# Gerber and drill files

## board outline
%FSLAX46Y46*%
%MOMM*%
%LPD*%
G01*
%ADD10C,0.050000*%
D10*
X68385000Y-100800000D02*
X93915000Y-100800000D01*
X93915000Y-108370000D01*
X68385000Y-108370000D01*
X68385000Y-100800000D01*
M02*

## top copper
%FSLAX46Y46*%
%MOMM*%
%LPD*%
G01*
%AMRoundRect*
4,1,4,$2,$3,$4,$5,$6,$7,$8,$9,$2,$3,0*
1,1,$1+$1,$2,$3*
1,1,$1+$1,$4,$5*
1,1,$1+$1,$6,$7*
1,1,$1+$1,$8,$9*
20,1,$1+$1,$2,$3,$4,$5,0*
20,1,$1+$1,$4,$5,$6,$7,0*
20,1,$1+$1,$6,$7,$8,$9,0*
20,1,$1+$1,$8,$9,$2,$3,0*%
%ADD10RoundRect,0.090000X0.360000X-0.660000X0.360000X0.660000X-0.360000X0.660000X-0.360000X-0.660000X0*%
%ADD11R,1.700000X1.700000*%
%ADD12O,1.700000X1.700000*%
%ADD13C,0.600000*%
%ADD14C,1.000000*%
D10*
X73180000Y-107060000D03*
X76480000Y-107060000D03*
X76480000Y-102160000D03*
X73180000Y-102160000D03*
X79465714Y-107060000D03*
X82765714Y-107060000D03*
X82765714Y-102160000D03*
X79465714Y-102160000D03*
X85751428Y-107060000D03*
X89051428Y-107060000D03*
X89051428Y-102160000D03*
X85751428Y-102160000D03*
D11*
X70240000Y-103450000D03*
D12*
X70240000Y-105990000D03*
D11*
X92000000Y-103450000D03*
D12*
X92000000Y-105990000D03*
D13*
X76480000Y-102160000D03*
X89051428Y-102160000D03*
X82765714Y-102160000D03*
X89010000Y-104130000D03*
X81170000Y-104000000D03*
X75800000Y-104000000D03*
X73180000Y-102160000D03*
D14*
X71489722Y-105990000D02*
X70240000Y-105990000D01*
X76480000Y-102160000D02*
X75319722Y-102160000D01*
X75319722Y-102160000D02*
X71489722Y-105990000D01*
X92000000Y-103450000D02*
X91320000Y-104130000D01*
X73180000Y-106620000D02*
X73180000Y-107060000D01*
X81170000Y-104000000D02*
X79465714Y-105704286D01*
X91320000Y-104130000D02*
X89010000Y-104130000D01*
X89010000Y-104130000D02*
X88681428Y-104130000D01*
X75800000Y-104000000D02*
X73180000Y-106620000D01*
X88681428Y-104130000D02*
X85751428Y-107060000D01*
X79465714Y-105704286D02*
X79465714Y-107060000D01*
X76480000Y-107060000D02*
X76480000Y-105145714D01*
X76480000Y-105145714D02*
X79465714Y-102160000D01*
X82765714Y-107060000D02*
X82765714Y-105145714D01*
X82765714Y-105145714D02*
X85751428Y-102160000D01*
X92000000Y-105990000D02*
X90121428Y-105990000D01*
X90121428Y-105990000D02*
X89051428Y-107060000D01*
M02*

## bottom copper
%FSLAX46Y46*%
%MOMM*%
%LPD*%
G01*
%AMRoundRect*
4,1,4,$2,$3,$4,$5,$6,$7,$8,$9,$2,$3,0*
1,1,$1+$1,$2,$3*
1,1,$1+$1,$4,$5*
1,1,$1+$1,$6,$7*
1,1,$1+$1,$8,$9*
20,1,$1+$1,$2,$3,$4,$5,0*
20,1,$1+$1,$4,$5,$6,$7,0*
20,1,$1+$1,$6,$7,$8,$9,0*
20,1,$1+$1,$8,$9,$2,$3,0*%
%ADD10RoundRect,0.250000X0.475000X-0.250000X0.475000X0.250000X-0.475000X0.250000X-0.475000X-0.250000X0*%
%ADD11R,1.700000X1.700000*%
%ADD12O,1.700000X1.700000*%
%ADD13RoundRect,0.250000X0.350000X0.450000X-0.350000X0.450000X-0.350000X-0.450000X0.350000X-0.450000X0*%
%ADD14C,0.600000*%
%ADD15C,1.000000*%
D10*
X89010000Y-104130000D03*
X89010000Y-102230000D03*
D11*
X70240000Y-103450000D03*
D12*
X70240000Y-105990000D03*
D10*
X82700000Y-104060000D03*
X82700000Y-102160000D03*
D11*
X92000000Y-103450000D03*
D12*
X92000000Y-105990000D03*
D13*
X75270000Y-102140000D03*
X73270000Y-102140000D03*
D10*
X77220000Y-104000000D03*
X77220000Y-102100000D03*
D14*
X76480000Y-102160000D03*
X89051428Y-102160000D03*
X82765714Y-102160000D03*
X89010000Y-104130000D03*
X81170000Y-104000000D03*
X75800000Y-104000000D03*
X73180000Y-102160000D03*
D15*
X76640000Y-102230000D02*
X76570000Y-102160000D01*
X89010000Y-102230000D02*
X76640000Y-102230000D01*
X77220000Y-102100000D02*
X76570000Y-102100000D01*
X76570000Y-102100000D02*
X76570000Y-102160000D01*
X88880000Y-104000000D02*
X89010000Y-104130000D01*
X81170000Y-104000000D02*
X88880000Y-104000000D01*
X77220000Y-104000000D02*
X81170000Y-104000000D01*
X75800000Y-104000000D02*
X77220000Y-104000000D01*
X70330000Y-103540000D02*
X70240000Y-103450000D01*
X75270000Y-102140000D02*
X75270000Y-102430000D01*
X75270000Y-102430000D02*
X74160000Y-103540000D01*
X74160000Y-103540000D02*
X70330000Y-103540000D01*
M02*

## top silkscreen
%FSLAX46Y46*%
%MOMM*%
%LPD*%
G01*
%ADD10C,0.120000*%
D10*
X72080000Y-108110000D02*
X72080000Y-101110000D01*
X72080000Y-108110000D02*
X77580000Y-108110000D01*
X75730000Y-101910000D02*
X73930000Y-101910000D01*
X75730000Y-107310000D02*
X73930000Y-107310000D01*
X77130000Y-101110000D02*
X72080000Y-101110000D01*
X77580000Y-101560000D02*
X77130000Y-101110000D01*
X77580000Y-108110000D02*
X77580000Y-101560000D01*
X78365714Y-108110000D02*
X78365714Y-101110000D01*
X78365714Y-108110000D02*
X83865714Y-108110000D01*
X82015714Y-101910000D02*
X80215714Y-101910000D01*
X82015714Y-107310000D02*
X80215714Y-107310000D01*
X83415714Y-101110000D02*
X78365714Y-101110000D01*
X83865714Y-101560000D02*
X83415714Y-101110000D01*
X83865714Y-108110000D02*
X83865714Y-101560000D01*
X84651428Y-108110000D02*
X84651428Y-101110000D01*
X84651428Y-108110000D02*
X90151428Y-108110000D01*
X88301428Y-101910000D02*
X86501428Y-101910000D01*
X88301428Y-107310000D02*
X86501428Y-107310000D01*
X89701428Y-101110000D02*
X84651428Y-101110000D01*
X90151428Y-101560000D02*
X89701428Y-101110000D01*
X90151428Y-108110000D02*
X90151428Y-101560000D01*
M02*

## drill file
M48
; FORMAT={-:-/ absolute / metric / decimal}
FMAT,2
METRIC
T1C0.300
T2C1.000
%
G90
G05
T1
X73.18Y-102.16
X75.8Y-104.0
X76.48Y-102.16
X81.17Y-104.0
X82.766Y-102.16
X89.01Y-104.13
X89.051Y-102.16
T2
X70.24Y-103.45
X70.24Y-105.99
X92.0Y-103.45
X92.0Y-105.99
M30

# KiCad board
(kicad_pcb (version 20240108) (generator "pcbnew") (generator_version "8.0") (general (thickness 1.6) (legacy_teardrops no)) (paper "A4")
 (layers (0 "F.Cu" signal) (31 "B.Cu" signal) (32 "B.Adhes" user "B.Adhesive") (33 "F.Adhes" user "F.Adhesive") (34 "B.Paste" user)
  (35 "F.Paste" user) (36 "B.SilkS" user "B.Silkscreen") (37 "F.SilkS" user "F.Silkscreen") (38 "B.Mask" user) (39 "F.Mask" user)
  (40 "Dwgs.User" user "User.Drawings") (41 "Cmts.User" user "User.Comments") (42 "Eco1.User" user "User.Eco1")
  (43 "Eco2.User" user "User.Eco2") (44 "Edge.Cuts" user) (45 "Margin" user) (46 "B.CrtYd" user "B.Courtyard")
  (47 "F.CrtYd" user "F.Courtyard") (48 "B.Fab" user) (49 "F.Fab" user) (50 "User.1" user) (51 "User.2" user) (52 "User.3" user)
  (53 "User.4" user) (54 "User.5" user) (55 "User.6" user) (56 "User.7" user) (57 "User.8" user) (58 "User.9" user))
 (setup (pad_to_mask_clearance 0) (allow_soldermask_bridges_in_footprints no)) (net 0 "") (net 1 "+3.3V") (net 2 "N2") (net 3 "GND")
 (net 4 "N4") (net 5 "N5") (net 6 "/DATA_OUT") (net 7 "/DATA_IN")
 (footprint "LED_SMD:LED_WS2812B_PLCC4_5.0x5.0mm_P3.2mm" (layer "F.Cu") (at 74.83 104.61 90)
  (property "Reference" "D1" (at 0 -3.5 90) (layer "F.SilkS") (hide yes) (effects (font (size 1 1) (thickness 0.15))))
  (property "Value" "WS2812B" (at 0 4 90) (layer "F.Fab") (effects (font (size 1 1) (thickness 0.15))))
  (fp_line (start -3.5 -2.75) (end 3.5 -2.75) (stroke (width 0.12) (type solid)) (layer "F.SilkS"))
  (fp_line (start -3.5 -2.75) (end -3.5 2.75) (stroke (width 0.12) (type default)) (layer "F.SilkS"))
  (fp_line (start 2.7 0.9) (end 2.7 -0.9) (stroke (width 0.12) (type default)) (layer "F.SilkS"))
  (fp_line (start -2.7 0.9) (end -2.7 -0.9) (stroke (width 0.12) (type default)) (layer "F.SilkS"))
  (fp_line (start 3.5 2.3) (end 3.5 -2.75) (stroke (width 0.12) (type default)) (layer "F.SilkS"))
  (fp_line (start 3.05 2.75) (end 3.5 2.3) (stroke (width 0.12) (type default)) (layer "F.SilkS"))
  (fp_line (start -3.5 2.75) (end 3.05 2.75) (stroke (width 0.12) (type solid)) (layer "F.SilkS"))
  (pad "1" smd roundrect (at -2.45 -1.65 90) (size 1.5 0.9) (layers "F.Cu" "F.Paste" "F.Mask") (roundrect_rratio 0.1) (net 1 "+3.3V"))
  (pad "2" smd roundrect (at -2.45 1.65 90) (size 1.5 0.9) (layers "F.Cu" "F.Paste" "F.Mask") (roundrect_rratio 0.1) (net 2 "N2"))
  (pad "3" smd roundrect (at 2.45 1.65 90) (size 1.5 0.9) (layers "F.Cu" "F.Paste" "F.Mask") (roundrect_rratio 0.1) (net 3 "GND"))
  (pad "4" smd roundrect (at 2.45 -1.65 90) (size 1.5 0.9) (layers "F.Cu" "F.Paste" "F.Mask") (roundrect_rratio 0.1) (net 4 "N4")))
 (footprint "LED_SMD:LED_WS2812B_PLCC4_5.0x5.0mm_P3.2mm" (layer "F.Cu") (at 81.115714 104.61 90)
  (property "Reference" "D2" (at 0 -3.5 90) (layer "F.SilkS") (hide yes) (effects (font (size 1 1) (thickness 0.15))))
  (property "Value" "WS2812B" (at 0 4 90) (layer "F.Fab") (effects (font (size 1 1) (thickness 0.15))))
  (fp_line (start -3.5 -2.75) (end 3.5 -2.75) (stroke (width 0.12) (type solid)) (layer "F.SilkS"))
  (fp_line (start -3.5 -2.75) (end -3.5 2.75) (stroke (width 0.12) (type default)) (layer "F.SilkS"))
  (fp_line (start 2.7 0.9) (end 2.7 -0.9) (stroke (width 0.12) (type default)) (layer "F.SilkS"))
  (fp_line (start -2.7 0.9) (end -2.7 -0.9) (stroke (width 0.12) (type default)) (layer "F.SilkS"))
  (fp_line (start 3.5 2.3) (end 3.5 -2.75) (stroke (width 0.12) (type default)) (layer "F.SilkS"))
  (fp_line (start 3.05 2.75) (end 3.5 2.3) (stroke (width 0.12) (type default)) (layer "F.SilkS"))
  (fp_line (start -3.5 2.75) (end 3.05 2.75) (stroke (width 0.12) (type solid)) (layer "F.SilkS"))
  (pad "1" smd roundrect (at -2.45 -1.65 90) (size 1.5 0.9) (layers "F.Cu" "F.Paste" "F.Mask") (roundrect_rratio 0.1) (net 1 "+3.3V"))
  (pad "2" smd roundrect (at -2.45 1.65 90) (size 1.5 0.9) (layers "F.Cu" "F.Paste" "F.Mask") (roundrect_rratio 0.1) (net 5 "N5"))
  (pad "3" smd roundrect (at 2.45 1.65 90) (size 1.5 0.9) (layers "F.Cu" "F.Paste" "F.Mask") (roundrect_rratio 0.1) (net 3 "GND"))
  (pad "4" smd roundrect (at 2.45 -1.65 90) (size 1.5 0.9) (layers "F.Cu" "F.Paste" "F.Mask") (roundrect_rratio 0.1) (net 2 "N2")))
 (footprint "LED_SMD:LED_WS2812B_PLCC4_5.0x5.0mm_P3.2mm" (layer "F.Cu") (at 87.401428 104.61 90)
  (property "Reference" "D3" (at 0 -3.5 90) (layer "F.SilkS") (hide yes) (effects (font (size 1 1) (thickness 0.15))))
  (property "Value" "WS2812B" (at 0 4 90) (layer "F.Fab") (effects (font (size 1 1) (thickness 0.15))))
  (fp_line (start -3.5 -2.75) (end 3.5 -2.75) (stroke (width 0.12) (type solid)) (layer "F.SilkS"))
  (fp_line (start -3.5 -2.75) (end -3.5 2.75) (stroke (width 0.12) (type default)) (layer "F.SilkS"))
  (fp_line (start 2.7 0.9) (end 2.7 -0.9) (stroke (width 0.12) (type default)) (layer "F.SilkS"))
  (fp_line (start -2.7 0.9) (end -2.7 -0.9) (stroke (width 0.12) (type default)) (layer "F.SilkS"))
  (fp_line (start 3.5 2.3) (end 3.5 -2.75) (stroke (width 0.12) (type default)) (layer "F.SilkS"))
  (fp_line (start 3.05 2.75) (end 3.5 2.3) (stroke (width 0.12) (type default)) (layer "F.SilkS"))
  (fp_line (start -3.5 2.75) (end 3.05 2.75) (stroke (width 0.12) (type solid)) (layer "F.SilkS"))
  (pad "1" smd roundrect (at -2.45 -1.65 90) (size 1.5 0.9) (layers "F.Cu" "F.Paste" "F.Mask") (roundrect_rratio 0.1) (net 1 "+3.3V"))
  (pad "2" smd roundrect (at -2.45 1.65 90) (size 1.5 0.9) (layers "F.Cu" "F.Paste" "F.Mask") (roundrect_rratio 0.1) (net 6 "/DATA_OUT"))
  (pad "3" smd roundrect (at 2.45 1.65 90) (size 1.5 0.9) (layers "F.Cu" "F.Paste" "F.Mask") (roundrect_rratio 0.1) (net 3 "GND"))
  (pad "4" smd roundrect (at 2.45 -1.65 90) (size 1.5 0.9) (layers "F.Cu" "F.Paste" "F.Mask") (roundrect_rratio 0.1) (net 5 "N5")))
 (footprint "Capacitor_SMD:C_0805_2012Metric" (layer "B.Cu") (at 89.01 103.18 90)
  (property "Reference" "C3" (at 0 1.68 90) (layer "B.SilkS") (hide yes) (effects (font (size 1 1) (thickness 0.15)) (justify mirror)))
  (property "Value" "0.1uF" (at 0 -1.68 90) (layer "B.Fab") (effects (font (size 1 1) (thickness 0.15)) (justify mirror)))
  (pad "1" smd roundrect (at -0.95 0 90) (size 1 1.45) (layers "B.Cu" "B.Paste" "B.Mask") (roundrect_rratio 0.25) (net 1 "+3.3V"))
  (pad "2" smd roundrect (at 0.95 0 90) (size 1 1.45) (layers "B.Cu" "B.Paste" "B.Mask") (roundrect_rratio 0.25) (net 3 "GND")))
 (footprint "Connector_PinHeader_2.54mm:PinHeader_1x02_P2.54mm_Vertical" (layer "B.Cu") (at 70.24 103.45 180)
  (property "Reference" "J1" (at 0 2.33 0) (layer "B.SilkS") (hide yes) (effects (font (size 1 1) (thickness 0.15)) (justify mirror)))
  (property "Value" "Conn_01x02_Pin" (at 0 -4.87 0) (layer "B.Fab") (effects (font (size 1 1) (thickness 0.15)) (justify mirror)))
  (pad "1" thru_hole rect (at 0 0 180) (size 1.7 1.7) (drill 1) (layers "*.Cu" "*.Mask") (remove_unused_layers no) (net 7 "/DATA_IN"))
  (pad "2" thru_hole oval (at 0 -2.54 180) (size 1.7 1.7) (drill 1) (layers "*.Cu" "*.Mask") (remove_unused_layers no) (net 3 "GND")))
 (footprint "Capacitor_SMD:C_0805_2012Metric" (layer "B.Cu") (at 82.7 103.11 90)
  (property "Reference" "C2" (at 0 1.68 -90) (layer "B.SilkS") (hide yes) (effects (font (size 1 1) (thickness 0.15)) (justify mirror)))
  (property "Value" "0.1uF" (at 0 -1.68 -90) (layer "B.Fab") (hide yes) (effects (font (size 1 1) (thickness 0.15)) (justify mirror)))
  (pad "1" smd roundrect (at -0.95 0 90) (size 1 1.45) (layers "B.Cu" "B.Paste" "B.Mask") (roundrect_rratio 0.25) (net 1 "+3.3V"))
  (pad "2" smd roundrect (at 0.95 0 90) (size 1 1.45) (layers "B.Cu" "B.Paste" "B.Mask") (roundrect_rratio 0.25) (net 3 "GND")))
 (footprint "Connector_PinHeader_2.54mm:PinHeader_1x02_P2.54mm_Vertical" (layer "B.Cu") (at 92 103.45 180)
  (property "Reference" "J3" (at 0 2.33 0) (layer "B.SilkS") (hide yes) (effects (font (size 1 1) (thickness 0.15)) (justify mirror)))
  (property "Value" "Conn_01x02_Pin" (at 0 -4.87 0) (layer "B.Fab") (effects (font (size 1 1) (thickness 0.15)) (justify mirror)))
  (pad "1" thru_hole rect (at 0 0 180) (size 1.7 1.7) (drill 1) (layers "*.Cu" "*.Mask") (remove_unused_layers no) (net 1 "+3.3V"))
  (pad "2" thru_hole oval (at 0 -2.54 180) (size 1.7 1.7) (drill 1) (layers "*.Cu" "*.Mask") (remove_unused_layers no) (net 6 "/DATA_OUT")))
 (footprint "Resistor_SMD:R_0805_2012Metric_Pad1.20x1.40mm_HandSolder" (layer "B.Cu") (at 74.27 102.14 180)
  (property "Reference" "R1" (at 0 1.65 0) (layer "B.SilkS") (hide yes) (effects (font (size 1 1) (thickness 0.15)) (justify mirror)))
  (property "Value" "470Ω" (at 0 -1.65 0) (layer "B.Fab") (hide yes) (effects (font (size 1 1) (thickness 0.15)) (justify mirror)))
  (pad "1" smd roundrect (at -1 0 180) (size 1.2 1.4) (layers "B.Cu" "B.Paste" "B.Mask") (roundrect_rratio 0.208333) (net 7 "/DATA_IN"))
  (pad "2" smd roundrect (at 1 0 180) (size 1.2 1.4) (layers "B.Cu" "B.Paste" "B.Mask") (roundrect_rratio 0.208333) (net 4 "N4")))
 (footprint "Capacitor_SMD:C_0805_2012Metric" (layer "B.Cu") (at 77.22 103.05 90)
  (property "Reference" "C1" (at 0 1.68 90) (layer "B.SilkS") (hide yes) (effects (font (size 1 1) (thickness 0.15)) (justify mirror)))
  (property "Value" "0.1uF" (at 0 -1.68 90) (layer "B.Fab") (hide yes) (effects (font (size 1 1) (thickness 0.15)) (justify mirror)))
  (pad "1" smd roundrect (at -0.95 0 90) (size 1 1.45) (layers "B.Cu" "B.Paste" "B.Mask") (roundrect_rratio 0.25) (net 1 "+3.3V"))
  (pad "2" smd roundrect (at 0.95 0 90) (size 1 1.45) (layers "B.Cu" "B.Paste" "B.Mask") (roundrect_rratio 0.25) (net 3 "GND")))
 (gr_rect (start 68.385 100.8) (end 93.915 108.37) (stroke (width 0.05) (type default)) (fill none) (layer "Edge.Cuts"))
 (segment (start 71.489722 105.99) (end 70.24 105.99) (width 1) (layer "F.Cu") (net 3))
 (segment (start 76.48 102.16) (end 75.319722 102.16) (width 1) (layer "F.Cu") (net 3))
 (segment (start 75.319722 102.16) (end 71.489722 105.99) (width 1) (layer "F.Cu") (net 3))
 (via (at 76.48 102.16) (size 0.6) (drill 0.3) (layers "F.Cu" "B.Cu") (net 3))
 (via (at 89.051428 102.16) (size 0.6) (drill 0.3) (layers "F.Cu" "B.Cu") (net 3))
 (via (at 82.765714 102.16) (size 0.6) (drill 0.3) (layers "F.Cu" "B.Cu") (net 3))
 (segment (start 76.64 102.23) (end 76.57 102.16) (width 1) (layer "B.Cu") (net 3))
 (segment (start 89.01 102.23) (end 76.64 102.23) (width 1) (layer "B.Cu") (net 3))
 (segment (start 77.22 102.1) (end 76.57 102.1) (width 1) (layer "B.Cu") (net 3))
 (segment (start 76.57 102.1) (end 76.57 102.16) (width 1) (layer "B.Cu") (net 3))
 (segment (start 92 103.45) (end 91.32 104.13) (width 1) (layer "F.Cu") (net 1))
 (segment (start 73.18 106.62) (end 73.18 107.06) (width 1) (layer "F.Cu") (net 1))
 (segment (start 81.17 104) (end 79.465714 105.704286) (width 1) (layer "F.Cu") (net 1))
 (segment (start 91.32 104.13) (end 89.01 104.13) (width 1) (layer "F.Cu") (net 1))
 (segment (start 89.01 104.13) (end 88.681428 104.13) (width 1) (layer "F.Cu") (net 1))
 (segment (start 75.8 104) (end 73.18 106.62) (width 1) (layer "F.Cu") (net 1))
 (segment (start 88.681428 104.13) (end 85.751428 107.06) (width 1) (layer "F.Cu") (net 1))
 (segment (start 79.465714 105.704286) (end 79.465714 107.06) (width 1) (layer "F.Cu") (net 1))
 (via (at 89.01 104.13) (size 0.6) (drill 0.3) (layers "F.Cu" "B.Cu") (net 1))
 (via (at 81.17 104) (size 0.6) (drill 0.3) (layers "F.Cu" "B.Cu") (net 1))
 (via (at 75.8 104) (size 0.6) (drill 0.3) (layers "F.Cu" "B.Cu") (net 1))
 (segment (start 88.88 104) (end 89.01 104.13) (width 1) (layer "B.Cu") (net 1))
 (segment (start 81.17 104) (end 88.88 104) (width 1) (layer "B.Cu") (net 1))
 (segment (start 77.22 104) (end 81.17 104) (width 1) (layer "B.Cu") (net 1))
 (segment (start 75.8 104) (end 77.22 104) (width 1) (layer "B.Cu") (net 1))
 (segment (start 76.48 107.06) (end 76.48 105.145714) (width 1) (layer "F.Cu") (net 2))
 (segment (start 76.48 105.145714) (end 79.465714 102.16) (width 1) (layer "F.Cu") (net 2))
 (via (at 73.18 102.16) (size 0.6) (drill 0.3) (layers "F.Cu" "B.Cu") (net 4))
 (segment (start 82.765714 107.06) (end 82.765714 105.145714) (width 1) (layer "F.Cu") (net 5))
 (segment (start 82.765714 105.145714) (end 85.751428 102.16) (width 1) (layer "F.Cu") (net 5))
 (segment (start 92 105.99) (end 90.121428 105.99) (width 1) (layer "F.Cu") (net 6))
 (segment (start 90.121428 105.99) (end 89.051428 107.06) (width 1) (layer "F.Cu") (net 6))
 (segment (start 70.33 103.54) (end 70.24 103.45) (width 1) (layer "B.Cu") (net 7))
 (segment (start 75.27 102.14) (end 75.27 102.43) (width 1) (layer "B.Cu") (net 7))
 (segment (start 75.27 102.43) (end 74.16 103.54) (width 1) (layer "B.Cu") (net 7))
 (segment (start 74.16 103.54) (end 70.33 103.54) (width 1) (layer "B.Cu") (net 7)))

